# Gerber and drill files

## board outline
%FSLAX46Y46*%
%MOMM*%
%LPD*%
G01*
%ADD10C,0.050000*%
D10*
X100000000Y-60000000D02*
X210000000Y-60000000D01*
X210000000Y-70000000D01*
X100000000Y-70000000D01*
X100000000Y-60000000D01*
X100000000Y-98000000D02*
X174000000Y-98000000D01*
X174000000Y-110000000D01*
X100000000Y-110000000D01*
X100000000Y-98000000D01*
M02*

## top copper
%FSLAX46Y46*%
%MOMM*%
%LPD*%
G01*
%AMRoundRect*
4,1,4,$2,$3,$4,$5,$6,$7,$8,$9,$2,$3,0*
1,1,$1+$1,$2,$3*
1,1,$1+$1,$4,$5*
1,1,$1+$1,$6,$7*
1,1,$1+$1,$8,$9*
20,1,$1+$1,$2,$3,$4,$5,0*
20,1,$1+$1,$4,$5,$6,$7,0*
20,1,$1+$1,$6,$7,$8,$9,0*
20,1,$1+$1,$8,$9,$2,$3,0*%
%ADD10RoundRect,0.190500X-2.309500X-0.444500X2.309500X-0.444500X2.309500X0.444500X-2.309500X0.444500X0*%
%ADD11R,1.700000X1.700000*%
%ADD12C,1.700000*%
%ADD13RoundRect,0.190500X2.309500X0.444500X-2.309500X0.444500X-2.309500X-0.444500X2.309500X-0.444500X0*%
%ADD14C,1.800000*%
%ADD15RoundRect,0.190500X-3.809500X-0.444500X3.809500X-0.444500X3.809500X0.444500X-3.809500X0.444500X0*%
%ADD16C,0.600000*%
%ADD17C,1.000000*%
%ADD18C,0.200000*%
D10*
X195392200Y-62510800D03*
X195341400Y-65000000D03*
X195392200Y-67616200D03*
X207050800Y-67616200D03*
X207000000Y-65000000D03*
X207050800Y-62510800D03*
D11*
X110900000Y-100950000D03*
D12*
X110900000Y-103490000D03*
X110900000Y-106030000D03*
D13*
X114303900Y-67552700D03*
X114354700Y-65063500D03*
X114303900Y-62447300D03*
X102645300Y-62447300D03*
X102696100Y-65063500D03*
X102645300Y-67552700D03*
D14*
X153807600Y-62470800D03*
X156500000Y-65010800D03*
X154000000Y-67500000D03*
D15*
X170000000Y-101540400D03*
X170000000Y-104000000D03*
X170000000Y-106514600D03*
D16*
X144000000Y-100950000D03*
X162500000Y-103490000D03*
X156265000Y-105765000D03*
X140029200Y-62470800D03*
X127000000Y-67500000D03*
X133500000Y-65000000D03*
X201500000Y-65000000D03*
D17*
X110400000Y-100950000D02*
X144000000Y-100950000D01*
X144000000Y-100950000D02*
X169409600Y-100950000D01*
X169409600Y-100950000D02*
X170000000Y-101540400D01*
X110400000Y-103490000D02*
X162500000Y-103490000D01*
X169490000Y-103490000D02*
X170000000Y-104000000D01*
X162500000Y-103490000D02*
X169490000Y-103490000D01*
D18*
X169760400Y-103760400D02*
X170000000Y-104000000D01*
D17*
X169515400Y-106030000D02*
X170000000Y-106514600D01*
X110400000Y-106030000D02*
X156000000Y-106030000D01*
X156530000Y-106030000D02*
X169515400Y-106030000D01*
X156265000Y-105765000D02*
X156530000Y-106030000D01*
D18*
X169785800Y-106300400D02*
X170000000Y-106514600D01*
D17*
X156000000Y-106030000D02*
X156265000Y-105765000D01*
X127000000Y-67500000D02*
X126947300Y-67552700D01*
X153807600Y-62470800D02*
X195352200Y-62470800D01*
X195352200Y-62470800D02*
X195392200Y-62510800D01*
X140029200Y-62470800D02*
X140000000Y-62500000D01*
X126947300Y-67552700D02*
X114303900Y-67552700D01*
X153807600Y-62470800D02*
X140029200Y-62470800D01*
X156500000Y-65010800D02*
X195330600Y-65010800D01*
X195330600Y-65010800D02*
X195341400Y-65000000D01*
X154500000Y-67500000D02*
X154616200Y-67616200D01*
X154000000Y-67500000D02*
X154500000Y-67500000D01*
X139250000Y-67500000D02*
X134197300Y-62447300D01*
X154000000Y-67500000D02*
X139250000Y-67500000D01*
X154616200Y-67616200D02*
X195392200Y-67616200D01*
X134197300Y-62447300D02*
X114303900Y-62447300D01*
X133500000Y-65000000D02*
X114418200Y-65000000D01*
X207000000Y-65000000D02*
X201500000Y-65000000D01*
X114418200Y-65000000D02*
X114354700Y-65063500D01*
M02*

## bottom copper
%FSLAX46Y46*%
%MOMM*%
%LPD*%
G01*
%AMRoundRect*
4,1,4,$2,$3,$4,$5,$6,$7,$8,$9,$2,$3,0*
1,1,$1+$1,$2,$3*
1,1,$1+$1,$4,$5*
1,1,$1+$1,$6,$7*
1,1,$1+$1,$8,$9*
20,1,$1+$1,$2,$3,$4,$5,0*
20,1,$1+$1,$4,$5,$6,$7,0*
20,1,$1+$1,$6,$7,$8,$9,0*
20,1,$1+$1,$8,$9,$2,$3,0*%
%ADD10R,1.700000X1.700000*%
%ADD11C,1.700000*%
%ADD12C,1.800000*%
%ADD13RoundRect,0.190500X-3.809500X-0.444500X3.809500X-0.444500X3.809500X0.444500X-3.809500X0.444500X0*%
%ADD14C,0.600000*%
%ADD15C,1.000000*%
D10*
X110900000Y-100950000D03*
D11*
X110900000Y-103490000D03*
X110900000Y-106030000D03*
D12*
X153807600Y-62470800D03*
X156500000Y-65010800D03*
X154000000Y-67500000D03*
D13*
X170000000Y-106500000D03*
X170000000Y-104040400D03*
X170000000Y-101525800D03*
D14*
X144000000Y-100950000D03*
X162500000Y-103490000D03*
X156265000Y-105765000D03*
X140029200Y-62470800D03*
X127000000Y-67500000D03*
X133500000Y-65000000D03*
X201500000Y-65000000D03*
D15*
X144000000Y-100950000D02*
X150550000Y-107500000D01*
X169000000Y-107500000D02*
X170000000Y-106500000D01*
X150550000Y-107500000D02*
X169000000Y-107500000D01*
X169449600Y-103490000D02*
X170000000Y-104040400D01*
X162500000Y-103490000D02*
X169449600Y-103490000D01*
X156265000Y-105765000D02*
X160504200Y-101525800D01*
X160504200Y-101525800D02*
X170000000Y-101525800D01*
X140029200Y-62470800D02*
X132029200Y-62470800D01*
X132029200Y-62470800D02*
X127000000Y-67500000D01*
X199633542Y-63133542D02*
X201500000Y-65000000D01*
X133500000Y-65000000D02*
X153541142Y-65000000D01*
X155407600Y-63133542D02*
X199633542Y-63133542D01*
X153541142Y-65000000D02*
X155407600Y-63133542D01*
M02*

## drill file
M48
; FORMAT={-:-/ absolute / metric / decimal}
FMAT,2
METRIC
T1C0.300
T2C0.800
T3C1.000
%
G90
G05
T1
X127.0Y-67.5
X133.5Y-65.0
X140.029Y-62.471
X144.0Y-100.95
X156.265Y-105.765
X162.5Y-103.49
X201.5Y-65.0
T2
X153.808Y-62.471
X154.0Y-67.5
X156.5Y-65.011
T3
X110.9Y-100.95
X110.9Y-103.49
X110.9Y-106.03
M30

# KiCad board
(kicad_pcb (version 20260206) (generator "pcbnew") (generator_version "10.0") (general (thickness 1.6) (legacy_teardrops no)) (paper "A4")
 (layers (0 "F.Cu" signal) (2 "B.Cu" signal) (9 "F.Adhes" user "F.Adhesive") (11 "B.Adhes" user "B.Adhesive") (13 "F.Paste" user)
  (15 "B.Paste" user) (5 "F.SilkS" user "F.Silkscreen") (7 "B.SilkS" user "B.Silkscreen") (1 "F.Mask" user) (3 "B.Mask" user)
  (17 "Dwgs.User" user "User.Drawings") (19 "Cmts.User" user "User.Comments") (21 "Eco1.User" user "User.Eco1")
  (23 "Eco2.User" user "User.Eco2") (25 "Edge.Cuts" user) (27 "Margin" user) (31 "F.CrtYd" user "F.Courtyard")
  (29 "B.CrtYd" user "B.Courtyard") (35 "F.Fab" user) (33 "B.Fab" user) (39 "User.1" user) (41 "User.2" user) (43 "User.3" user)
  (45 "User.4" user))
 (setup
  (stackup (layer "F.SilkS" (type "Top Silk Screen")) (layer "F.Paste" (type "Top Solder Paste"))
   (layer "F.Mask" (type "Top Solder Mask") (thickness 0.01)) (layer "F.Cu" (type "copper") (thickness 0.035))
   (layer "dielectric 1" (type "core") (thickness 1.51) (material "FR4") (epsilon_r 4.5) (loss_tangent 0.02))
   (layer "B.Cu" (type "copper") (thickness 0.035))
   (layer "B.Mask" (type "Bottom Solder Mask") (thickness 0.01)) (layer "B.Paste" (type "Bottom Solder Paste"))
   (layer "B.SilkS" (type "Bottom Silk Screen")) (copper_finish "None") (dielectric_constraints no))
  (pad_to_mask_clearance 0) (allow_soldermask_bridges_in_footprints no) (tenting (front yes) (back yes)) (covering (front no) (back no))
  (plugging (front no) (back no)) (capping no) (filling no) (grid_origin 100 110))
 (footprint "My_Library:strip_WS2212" (layer "F.Cu") (at 200.4468 62.46)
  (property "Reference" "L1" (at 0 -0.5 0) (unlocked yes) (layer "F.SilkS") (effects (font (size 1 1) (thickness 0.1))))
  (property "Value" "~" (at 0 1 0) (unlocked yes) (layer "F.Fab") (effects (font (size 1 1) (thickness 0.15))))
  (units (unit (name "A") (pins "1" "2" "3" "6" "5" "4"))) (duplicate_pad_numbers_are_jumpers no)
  (pad "1" smd roundrect (at -5.0546 0.0508) (size 5 1.27) (layers "F.Cu" "F.Mask") (roundrect_rratio 0.15) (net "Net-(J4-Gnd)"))
  (pad "2" smd roundrect (at -5.1054 2.54) (size 5 1.27) (layers "F.Cu" "F.Mask") (roundrect_rratio 0.15) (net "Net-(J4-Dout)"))
  (pad "3" smd roundrect (at -5.0546 5.1562) (size 5 1.27) (layers "F.Cu" "F.Mask") (roundrect_rratio 0.15) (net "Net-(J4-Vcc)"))
  (pad "4" smd roundrect (at 6.604 5.1562) (size 5 1.27) (layers "F.Cu" "F.Mask") (roundrect_rratio 0.15) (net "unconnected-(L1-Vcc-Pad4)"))
  (pad "5" smd roundrect (at 6.5532 2.54) (size 5 1.27) (layers "F.Cu" "F.Mask") (roundrect_rratio 0.15) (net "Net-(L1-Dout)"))
  (pad "6" smd roundrect (at 6.604 0.0508) (size 5 1.27) (layers "F.Cu" "F.Mask") (roundrect_rratio 0.15) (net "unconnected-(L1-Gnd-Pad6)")))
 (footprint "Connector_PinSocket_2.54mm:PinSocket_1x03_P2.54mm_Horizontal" (layer "F.Cu") (at 110.9 100.95)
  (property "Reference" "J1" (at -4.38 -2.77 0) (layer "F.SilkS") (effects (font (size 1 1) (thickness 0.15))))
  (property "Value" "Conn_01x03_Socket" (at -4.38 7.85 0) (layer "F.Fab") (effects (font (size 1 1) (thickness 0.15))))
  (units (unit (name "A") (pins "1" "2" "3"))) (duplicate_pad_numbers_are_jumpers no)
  (pad "1" thru_hole rect (at 0 0) (size 1.7 1.7) (drill 1) (layers "*.Cu" "*.Mask") (remove_unused_layers no) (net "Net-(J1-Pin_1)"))
  (pad "2" thru_hole circle (at 0 2.54) (size 1.7 1.7) (drill 1) (layers "*.Cu" "*.Mask") (remove_unused_layers no) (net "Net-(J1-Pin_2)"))
  (pad "3" thru_hole circle (at 0 5.08) (size 1.7 1.7) (drill 1) (layers "*.Cu" "*.Mask") (remove_unused_layers no) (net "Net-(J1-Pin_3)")))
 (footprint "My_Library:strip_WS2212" (layer "F.Cu") (at 109.2493 67.6035 180)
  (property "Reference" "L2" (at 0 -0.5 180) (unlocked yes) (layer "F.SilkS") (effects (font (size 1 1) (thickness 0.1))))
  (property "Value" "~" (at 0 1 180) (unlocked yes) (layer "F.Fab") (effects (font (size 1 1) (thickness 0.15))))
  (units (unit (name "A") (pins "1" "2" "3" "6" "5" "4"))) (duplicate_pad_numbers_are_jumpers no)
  (pad "1" smd roundrect (at -5.0546 0.0508 180) (size 5 1.27) (layers "F.Cu" "F.Mask") (roundrect_rratio 0.15) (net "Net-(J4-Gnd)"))
  (pad "2" smd roundrect (at -5.1054 2.54 180) (size 5 1.27) (layers "F.Cu" "F.Mask") (roundrect_rratio 0.15) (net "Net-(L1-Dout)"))
  (pad "3" smd roundrect (at -5.0546 5.1562 180) (size 5 1.27) (layers "F.Cu" "F.Mask") (roundrect_rratio 0.15) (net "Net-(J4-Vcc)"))
  (pad "4" smd roundrect (at 6.604 5.1562 180) (size 5 1.27) (layers "F.Cu" "F.Mask") (roundrect_rratio 0.15)
   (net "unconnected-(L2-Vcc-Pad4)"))
  (pad "5" smd roundrect (at 6.5532 2.54 180) (size 5 1.27) (layers "F.Cu" "F.Mask") (roundrect_rratio 0.15)
   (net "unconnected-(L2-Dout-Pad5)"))
  (pad "6" smd roundrect (at 6.604 0.0508 180) (size 5 1.27) (layers "F.Cu" "F.Mask") (roundrect_rratio 0.15)
   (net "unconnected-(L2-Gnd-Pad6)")))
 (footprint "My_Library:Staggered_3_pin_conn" (layer "F.Cu") (at 156.3476 57.3654)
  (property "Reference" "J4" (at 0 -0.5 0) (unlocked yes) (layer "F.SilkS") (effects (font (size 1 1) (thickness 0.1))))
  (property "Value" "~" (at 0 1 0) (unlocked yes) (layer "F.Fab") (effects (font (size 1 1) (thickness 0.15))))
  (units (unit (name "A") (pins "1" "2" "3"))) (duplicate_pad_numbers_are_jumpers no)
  (pad "1" thru_hole circle (at -2.54 5.1054) (size 1.8 1.8) (drill 0.8) (layers "*.Cu" "F.Mask") (remove_unused_layers no)
   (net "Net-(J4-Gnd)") (thermal_bridge_angle 90))
  (pad "2" thru_hole circle (at 0.1524 7.6454) (size 1.8 1.8) (drill 0.8) (layers "*.Cu" "F.Mask") (remove_unused_layers no)
   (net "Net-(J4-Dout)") (thermal_bridge_angle 90))
  (pad "3" thru_hole circle (at -2.3476 10.1346) (size 1.8 1.8) (drill 0.8) (layers "*.Cu" "F.Mask") (remove_unused_layers no)
   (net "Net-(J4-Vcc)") (thermal_bridge_angle 90)))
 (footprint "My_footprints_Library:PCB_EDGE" (layer "F.Cu") (at 170 97.0404)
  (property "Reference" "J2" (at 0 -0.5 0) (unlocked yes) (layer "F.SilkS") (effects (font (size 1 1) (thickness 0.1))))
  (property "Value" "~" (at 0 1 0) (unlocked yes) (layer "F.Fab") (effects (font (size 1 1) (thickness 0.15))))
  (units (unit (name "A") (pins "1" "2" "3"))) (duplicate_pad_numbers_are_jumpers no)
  (pad "1" smd roundrect (at 0 4.5) (size 8 1.27) (layers "F.Cu" "F.Mask" "F.Paste") (roundrect_rratio 0.15) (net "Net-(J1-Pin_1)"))
  (pad "2" smd roundrect (at 0 6.9596) (size 8 1.27) (layers "F.Cu" "F.Mask" "F.Paste") (roundrect_rratio 0.15) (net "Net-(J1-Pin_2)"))
  (pad "3" smd roundrect (at 0 9.4742) (size 8 1.27) (layers "F.Cu" "F.Mask" "F.Paste") (roundrect_rratio 0.15) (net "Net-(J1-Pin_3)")))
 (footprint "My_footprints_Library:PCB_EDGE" (layer "B.Cu") (at 170 111)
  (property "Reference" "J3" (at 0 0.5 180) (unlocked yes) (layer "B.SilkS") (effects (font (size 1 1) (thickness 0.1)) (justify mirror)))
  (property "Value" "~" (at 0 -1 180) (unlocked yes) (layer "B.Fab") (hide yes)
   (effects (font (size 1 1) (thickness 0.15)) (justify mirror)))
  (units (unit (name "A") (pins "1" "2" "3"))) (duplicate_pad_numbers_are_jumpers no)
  (pad "1" smd roundrect (at 0 -4.5) (size 8 1.27) (layers "B.Cu" "B.Mask" "B.Paste") (roundrect_rratio 0.15) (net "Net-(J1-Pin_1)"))
  (pad "2" smd roundrect (at 0 -6.9596) (size 8 1.27) (layers "B.Cu" "B.Mask" "B.Paste") (roundrect_rratio 0.15) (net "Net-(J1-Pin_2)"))
  (pad "3" smd roundrect (at 0 -9.4742) (size 8 1.27) (layers "B.Cu" "B.Mask" "B.Paste") (roundrect_rratio 0.15) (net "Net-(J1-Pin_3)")))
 (gr_rect (start 100 60) (end 210 70) (stroke (width 0.05) (type default)) (fill no) (layer "Edge.Cuts"))
 (gr_rect (start 100 98) (end 174 110) (stroke (width 0.05) (type default)) (fill no) (layer "Edge.Cuts"))
 (segment (start 110.4 100.95) (end 144 100.95) (width 1) (layer "F.Cu") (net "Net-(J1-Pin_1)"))
 (segment (start 144 100.95) (end 169.4096 100.95) (width 1) (layer "F.Cu") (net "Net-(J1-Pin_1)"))
 (segment (start 169.4096 100.95) (end 170 101.5404) (width 1) (layer "F.Cu") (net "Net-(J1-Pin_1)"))
 (via (at 144 100.95) (size 0.6) (drill 0.3) (layers "F.Cu" "B.Cu") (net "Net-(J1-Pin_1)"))
 (segment (start 144 100.95) (end 150.55 107.5) (width 1) (layer "B.Cu") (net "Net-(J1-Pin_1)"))
 (segment (start 169 107.5) (end 170 106.5) (width 1) (layer "B.Cu") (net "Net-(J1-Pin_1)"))
 (segment (start 150.55 107.5) (end 169 107.5) (width 1) (layer "B.Cu") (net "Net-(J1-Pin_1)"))
 (segment (start 110.4 103.49) (end 162.5 103.49) (width 1) (layer "F.Cu") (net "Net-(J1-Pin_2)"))
 (segment (start 169.49 103.49) (end 170 104) (width 1) (layer "F.Cu") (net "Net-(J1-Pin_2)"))
 (segment (start 162.5 103.49) (end 169.49 103.49) (width 1) (layer "F.Cu") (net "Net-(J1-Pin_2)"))
 (segment (start 169.7604 103.7604) (end 170 104) (width 0.2) (layer "F.Cu") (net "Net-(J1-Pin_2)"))
 (via (at 162.5 103.49) (size 0.6) (drill 0.3) (layers "F.Cu" "B.Cu") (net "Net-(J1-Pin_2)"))
 (segment (start 169.4496 103.49) (end 170 104.0404) (width 1) (layer "B.Cu") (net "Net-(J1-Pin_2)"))
 (segment (start 162.5 103.49) (end 169.4496 103.49) (width 1) (layer "B.Cu") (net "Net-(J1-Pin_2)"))
 (segment (start 169.5154 106.03) (end 170 106.5146) (width 1) (layer "F.Cu") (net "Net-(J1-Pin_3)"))
 (segment (start 110.4 106.03) (end 156 106.03) (width 1) (layer "F.Cu") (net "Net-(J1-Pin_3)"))
 (segment (start 156.53 106.03) (end 169.5154 106.03) (width 1) (layer "F.Cu") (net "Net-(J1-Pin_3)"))
 (segment (start 156.265 105.765) (end 156.53 106.03) (width 1) (layer "F.Cu") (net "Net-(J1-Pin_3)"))
 (segment (start 169.7858 106.3004) (end 170 106.5146) (width 0.2) (layer "F.Cu") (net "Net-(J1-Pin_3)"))
 (segment (start 156 106.03) (end 156.265 105.765) (width 1) (layer "F.Cu") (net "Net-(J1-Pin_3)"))
 (via (at 156.265 105.765) (size 0.6) (drill 0.3) (layers "F.Cu" "B.Cu") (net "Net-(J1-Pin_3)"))
 (segment (start 156.265 105.765) (end 160.5042 101.5258) (width 1) (layer "B.Cu") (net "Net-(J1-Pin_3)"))
 (segment (start 160.5042 101.5258) (end 170 101.5258) (width 1) (layer "B.Cu") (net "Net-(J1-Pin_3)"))
 (segment (start 127 67.5) (end 126.9473 67.5527) (width 1) (layer "F.Cu") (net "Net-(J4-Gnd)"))
 (segment (start 153.8076 62.4708) (end 195.3522 62.4708) (width 1) (layer "F.Cu") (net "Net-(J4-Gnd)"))
 (segment (start 195.3522 62.4708) (end 195.3922 62.5108) (width 1) (layer "F.Cu") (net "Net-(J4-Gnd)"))
 (segment (start 140.0292 62.4708) (end 140 62.5) (width 1) (layer "F.Cu") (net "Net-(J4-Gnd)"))
 (segment (start 126.9473 67.5527) (end 114.3039 67.5527) (width 1) (layer "F.Cu") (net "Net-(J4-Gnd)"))
 (segment (start 153.8076 62.4708) (end 140.0292 62.4708) (width 1) (layer "F.Cu") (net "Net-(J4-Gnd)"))
 (via (at 140.0292 62.4708) (size 0.6) (drill 0.3) (layers "F.Cu" "B.Cu") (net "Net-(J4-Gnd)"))
 (via (at 127 67.5) (size 0.6) (drill 0.3) (layers "F.Cu" "B.Cu") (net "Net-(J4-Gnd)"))
 (segment (start 140.0292 62.4708) (end 132.0292 62.4708) (width 1) (layer "B.Cu") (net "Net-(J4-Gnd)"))
 (segment (start 132.0292 62.4708) (end 127 67.5) (width 1) (layer "B.Cu") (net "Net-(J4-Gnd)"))
 (segment (start 156.5 65.0108) (end 195.3306 65.0108) (width 1) (layer "F.Cu") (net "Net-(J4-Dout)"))
 (segment (start 195.3306 65.0108) (end 195.3414 65) (width 1) (layer "F.Cu") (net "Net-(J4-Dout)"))
 (segment (start 154.5 67.5) (end 154.6162 67.6162) (width 1) (layer "F.Cu") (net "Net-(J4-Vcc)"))
 (segment (start 154 67.5) (end 154.5 67.5) (width 1) (layer "F.Cu") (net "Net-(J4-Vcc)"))
 (segment (start 139.25 67.5) (end 134.1973 62.4473) (width 1) (layer "F.Cu") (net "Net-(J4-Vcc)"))
 (segment (start 154 67.5) (end 139.25 67.5) (width 1) (layer "F.Cu") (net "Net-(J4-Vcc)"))
 (segment (start 154.6162 67.6162) (end 195.3922 67.6162) (width 1) (layer "F.Cu") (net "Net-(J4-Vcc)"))
 (segment (start 134.1973 62.4473) (end 114.3039 62.4473) (width 1) (layer "F.Cu") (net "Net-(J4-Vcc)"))
 (segment (start 133.5 65) (end 114.4182 65) (width 1) (layer "F.Cu") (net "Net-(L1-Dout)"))
 (segment (start 207 65) (end 201.5 65) (width 1) (layer "F.Cu") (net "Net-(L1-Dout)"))
 (segment (start 114.4182 65) (end 114.3547 65.0635) (width 1) (layer "F.Cu") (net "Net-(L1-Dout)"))
 (via (at 133.5 65) (size 0.6) (drill 0.3) (layers "F.Cu" "B.Cu") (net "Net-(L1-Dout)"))
 (via (at 201.5 65) (size 0.6) (drill 0.3) (layers "F.Cu" "B.Cu") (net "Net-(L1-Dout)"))
 (segment (start 199.633542 63.133542) (end 201.5 65) (width 1) (layer "B.Cu") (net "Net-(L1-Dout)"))
 (segment (start 133.5 65) (end 153.541142 65) (width 1) (layer "B.Cu") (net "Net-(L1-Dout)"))
 (segment (start 155.4076 63.133542) (end 199.633542 63.133542) (width 1) (layer "B.Cu") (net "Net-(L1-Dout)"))
 (segment (start 153.541142 65) (end 155.4076 63.133542) (width 1) (layer "B.Cu") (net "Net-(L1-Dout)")))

